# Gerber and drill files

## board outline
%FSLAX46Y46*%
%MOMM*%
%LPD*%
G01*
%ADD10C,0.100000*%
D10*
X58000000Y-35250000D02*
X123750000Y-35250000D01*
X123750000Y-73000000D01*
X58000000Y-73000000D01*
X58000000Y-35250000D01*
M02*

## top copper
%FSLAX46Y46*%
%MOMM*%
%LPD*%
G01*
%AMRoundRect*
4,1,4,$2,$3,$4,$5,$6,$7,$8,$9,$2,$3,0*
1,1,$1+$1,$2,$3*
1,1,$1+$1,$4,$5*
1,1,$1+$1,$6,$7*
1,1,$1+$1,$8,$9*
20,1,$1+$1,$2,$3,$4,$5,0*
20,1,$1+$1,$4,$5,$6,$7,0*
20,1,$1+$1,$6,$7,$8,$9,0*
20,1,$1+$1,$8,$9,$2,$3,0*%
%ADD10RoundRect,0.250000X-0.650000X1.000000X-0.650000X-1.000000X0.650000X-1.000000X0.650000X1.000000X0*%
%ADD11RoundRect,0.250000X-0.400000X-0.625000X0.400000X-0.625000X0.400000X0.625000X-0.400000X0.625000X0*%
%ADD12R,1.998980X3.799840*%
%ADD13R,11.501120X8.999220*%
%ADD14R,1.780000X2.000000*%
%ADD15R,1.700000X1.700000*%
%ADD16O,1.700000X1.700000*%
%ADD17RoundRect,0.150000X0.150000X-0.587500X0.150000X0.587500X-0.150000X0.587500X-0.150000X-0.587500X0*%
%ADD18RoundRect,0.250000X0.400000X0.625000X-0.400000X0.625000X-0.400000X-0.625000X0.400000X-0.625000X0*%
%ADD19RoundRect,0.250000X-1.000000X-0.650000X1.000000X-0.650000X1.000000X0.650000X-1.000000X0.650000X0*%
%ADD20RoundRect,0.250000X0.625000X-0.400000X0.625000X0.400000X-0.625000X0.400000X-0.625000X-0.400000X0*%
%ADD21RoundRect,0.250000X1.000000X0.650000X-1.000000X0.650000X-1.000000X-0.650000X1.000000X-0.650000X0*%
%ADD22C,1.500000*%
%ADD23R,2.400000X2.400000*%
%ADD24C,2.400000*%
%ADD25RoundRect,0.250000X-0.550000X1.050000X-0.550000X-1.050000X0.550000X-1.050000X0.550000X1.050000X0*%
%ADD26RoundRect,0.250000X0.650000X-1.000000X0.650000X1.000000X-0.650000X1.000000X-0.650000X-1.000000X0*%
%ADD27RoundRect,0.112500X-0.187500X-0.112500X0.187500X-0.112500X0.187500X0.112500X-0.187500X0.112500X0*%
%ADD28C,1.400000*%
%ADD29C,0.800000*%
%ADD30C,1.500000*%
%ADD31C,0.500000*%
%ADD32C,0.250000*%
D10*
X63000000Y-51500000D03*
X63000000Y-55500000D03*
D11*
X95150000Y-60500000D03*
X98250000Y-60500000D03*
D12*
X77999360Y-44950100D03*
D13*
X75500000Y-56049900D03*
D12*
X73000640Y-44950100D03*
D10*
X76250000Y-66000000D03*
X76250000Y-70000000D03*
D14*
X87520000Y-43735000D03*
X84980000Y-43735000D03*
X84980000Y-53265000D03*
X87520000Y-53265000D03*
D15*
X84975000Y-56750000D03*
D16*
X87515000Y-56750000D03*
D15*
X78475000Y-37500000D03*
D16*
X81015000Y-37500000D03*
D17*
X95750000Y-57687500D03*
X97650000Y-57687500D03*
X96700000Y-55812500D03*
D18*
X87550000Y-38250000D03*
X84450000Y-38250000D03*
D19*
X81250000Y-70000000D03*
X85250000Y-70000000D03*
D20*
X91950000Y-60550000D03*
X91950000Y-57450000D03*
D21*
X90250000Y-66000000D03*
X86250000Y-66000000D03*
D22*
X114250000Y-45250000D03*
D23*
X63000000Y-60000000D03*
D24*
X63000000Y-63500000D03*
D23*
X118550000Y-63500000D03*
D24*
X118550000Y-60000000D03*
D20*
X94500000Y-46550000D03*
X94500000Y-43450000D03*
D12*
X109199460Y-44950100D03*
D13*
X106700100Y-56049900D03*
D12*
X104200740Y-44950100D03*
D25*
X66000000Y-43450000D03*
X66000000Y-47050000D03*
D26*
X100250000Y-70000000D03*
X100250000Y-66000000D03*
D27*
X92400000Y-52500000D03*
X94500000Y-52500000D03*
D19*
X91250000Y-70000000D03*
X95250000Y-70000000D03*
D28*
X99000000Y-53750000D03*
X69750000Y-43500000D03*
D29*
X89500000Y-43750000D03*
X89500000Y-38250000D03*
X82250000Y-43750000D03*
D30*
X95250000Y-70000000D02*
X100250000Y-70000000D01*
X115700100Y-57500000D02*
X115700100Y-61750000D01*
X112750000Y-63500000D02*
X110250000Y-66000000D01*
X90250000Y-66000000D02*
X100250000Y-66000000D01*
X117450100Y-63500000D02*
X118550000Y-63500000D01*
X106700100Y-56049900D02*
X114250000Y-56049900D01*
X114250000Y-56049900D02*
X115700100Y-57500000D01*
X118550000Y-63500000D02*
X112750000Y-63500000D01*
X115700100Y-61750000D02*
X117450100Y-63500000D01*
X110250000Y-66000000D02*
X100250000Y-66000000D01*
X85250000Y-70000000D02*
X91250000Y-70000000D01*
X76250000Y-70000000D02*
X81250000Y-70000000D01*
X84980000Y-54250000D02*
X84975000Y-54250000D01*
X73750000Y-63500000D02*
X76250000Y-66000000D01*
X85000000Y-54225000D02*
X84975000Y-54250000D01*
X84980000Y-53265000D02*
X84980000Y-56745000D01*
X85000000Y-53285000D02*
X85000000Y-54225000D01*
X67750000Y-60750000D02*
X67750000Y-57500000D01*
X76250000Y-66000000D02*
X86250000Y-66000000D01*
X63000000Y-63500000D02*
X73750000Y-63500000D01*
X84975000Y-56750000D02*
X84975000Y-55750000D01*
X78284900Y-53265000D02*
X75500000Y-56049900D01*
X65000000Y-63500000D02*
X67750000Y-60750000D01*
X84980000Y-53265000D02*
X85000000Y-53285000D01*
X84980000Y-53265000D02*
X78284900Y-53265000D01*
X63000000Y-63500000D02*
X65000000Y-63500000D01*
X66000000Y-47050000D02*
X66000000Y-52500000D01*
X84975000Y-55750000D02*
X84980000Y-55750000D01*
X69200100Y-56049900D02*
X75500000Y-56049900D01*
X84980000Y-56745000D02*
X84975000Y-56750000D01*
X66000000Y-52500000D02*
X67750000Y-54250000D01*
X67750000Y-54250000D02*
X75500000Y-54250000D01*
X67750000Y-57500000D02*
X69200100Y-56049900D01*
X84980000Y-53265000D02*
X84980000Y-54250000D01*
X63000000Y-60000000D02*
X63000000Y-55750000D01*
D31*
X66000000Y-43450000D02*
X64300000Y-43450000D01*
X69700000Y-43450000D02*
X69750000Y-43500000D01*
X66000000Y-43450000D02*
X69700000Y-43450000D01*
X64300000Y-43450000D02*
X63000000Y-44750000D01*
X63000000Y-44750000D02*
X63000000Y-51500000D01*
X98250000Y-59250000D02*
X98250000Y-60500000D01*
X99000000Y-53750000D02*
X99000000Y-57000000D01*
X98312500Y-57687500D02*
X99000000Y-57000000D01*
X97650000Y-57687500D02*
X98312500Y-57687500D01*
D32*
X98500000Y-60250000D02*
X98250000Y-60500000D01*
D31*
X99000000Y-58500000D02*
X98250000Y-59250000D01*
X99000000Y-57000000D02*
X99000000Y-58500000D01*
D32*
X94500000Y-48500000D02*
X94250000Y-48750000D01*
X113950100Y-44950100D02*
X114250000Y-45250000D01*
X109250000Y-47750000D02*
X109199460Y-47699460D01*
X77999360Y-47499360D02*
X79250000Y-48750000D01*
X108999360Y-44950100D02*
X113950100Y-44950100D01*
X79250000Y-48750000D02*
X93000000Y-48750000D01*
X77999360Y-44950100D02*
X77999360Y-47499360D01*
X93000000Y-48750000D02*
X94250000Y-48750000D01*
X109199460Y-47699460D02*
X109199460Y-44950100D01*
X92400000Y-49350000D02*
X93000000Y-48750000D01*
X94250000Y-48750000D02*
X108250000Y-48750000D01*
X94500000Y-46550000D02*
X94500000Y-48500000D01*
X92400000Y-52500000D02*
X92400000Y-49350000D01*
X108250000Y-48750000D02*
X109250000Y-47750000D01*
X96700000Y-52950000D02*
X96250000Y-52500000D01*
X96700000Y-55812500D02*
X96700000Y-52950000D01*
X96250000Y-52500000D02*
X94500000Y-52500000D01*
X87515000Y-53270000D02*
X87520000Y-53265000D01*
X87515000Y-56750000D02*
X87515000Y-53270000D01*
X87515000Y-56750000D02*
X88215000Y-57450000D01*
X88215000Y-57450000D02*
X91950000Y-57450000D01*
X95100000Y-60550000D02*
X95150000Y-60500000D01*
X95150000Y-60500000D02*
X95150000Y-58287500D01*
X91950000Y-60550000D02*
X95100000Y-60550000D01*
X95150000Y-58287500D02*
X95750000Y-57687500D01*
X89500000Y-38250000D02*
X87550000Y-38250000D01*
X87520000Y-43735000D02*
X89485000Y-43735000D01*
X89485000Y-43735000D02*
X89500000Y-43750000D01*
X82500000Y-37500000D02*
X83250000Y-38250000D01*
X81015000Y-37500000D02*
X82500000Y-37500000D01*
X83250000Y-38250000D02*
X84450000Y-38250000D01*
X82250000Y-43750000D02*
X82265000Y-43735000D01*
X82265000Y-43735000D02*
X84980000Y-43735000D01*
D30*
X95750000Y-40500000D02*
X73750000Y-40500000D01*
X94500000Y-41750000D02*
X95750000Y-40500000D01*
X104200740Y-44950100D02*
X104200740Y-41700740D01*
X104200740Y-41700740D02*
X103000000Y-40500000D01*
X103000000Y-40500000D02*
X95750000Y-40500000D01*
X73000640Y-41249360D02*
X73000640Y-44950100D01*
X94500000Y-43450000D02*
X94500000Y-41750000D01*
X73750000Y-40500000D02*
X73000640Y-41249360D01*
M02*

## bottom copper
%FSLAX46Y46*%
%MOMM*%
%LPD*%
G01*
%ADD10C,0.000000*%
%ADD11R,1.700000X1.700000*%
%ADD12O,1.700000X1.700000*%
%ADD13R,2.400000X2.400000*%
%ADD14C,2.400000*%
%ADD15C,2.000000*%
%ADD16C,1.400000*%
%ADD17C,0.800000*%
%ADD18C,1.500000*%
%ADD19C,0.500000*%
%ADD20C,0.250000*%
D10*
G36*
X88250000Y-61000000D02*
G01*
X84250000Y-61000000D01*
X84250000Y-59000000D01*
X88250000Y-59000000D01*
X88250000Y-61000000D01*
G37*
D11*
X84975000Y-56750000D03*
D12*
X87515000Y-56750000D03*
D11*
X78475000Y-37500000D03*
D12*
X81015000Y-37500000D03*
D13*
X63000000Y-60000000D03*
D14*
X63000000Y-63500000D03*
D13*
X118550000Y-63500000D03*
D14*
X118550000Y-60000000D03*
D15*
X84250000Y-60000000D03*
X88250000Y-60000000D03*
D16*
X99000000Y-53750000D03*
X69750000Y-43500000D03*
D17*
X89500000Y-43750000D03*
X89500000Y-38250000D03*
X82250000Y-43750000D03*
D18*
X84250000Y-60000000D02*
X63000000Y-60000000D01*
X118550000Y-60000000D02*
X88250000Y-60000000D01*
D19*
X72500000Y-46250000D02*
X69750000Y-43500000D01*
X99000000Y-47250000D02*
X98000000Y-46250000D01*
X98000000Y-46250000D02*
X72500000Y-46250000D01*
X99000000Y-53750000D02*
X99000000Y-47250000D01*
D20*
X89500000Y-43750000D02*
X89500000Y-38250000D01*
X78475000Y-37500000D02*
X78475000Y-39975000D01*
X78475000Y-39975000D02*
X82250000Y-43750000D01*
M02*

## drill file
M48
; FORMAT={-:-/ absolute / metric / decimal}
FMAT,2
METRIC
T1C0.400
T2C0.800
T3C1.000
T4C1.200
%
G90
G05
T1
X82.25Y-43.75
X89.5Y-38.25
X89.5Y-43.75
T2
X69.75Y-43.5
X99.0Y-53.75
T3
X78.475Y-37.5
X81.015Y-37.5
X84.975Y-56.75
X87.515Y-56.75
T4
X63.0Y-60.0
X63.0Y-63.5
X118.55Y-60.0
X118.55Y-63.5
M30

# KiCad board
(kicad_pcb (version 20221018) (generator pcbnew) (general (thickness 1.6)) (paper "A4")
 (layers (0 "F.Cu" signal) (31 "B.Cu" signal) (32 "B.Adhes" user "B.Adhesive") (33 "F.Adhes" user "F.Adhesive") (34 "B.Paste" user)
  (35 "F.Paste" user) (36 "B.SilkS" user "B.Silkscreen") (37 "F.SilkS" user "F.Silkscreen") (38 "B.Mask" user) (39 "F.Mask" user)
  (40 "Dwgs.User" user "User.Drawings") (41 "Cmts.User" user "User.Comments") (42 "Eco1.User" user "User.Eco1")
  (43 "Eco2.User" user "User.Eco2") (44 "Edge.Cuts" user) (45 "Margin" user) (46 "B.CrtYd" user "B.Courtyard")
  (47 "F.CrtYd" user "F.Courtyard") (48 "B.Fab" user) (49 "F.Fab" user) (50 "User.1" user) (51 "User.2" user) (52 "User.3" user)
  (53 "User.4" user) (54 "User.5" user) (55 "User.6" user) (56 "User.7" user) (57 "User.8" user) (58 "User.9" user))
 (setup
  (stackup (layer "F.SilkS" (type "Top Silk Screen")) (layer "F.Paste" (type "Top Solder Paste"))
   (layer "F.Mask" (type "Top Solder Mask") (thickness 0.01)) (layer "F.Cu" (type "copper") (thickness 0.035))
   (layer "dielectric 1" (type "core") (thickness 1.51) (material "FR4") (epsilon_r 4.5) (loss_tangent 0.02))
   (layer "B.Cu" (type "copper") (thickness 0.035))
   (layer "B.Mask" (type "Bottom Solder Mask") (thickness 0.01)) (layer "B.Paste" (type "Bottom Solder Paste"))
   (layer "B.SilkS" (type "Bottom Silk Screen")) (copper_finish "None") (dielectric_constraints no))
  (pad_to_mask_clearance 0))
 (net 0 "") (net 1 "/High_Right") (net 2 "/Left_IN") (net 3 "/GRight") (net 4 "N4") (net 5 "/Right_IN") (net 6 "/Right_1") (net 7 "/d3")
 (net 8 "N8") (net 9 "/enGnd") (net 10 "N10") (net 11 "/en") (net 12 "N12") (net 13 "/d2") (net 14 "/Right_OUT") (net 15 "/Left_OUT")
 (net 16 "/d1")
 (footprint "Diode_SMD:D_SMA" (layer "F.Cu") (at 63 53.5 -90)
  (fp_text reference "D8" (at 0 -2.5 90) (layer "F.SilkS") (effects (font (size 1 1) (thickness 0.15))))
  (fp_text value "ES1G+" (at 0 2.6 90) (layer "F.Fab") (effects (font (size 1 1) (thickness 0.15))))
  (pad "1" smd roundrect (at -2 0 270) (size 2.5 1.8) (layers "F.Cu" "F.Paste" "F.Mask") (roundrect_rratio 0.1388888889)
   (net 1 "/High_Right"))
  (pad "2" smd roundrect (at 2 0 270) (size 2.5 1.8) (layers "F.Cu" "F.Paste" "F.Mask") (roundrect_rratio 0.1388888889) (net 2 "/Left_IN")))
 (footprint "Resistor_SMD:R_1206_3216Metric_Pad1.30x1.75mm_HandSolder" (layer "F.Cu") (at 96.7 60.5)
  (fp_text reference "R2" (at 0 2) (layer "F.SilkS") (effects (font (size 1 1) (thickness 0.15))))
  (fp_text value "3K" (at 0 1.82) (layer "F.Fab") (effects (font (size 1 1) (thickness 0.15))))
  (pad "1" smd roundrect (at -1.55 0) (size 1.3 1.75) (layers "F.Cu" "F.Paste" "F.Mask") (roundrect_rratio 0.192308) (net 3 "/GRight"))
  (pad "2" smd roundrect (at 1.55 0) (size 1.3 1.75) (layers "F.Cu" "F.Paste" "F.Mask") (roundrect_rratio 0.192308) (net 1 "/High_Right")))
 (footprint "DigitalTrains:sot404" (layer "F.Cu") (at 75.5 50.5 180)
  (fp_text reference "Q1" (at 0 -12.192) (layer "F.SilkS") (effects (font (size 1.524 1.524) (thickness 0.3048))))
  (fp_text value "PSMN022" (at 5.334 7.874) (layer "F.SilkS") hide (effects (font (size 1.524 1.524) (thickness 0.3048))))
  (pad "1" smd rect (at -2.49936 5.5499 180) (size 1.99898 3.79984) (layers "F.Cu" "F.Paste" "F.Mask") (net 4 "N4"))
  (pad "2" smd rect (at 0 -5.5499 180) (size 11.50112 8.99922) (layers "F.Cu" "F.Paste" "F.Mask") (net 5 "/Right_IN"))
  (pad "3" smd rect (at 2.49936 5.5499 180) (size 1.99898 3.79984) (layers "F.Cu" "F.Paste" "F.Mask") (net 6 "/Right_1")))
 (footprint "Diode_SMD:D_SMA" (layer "F.Cu") (at 76.25 68 -90)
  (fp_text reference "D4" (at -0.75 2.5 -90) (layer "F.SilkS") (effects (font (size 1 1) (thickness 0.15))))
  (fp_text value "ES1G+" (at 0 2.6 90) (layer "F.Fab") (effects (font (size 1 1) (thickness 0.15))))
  (pad "1" smd roundrect (at -2 0 270) (size 2.5 1.8) (layers "F.Cu" "F.Paste" "F.Mask") (roundrect_rratio 0.1388888889) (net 5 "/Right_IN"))
  (pad "2" smd roundrect (at 2 0 270) (size 2.5 1.8) (layers "F.Cu" "F.Paste" "F.Mask") (roundrect_rratio 0.1388888889) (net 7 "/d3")))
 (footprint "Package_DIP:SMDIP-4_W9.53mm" (layer "F.Cu") (at 86.25 48.5 -90)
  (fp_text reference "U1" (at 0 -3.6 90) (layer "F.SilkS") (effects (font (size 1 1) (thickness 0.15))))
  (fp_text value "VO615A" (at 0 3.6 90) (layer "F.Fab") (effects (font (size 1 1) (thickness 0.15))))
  (pad "1" smd rect (at -4.765 -1.27 270) (size 2 1.78) (layers "F.Cu" "F.Paste" "F.Mask") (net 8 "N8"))
  (pad "2" smd rect (at -4.765 1.27 270) (size 2 1.78) (layers "F.Cu" "F.Paste" "F.Mask") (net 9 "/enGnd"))
  (pad "3" smd rect (at 4.765 1.27 270) (size 2 1.78) (layers "F.Cu" "F.Paste" "F.Mask") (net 5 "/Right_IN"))
  (pad "4" smd rect (at 4.765 -1.27 270) (size 2 1.78) (layers "F.Cu" "F.Paste" "F.Mask") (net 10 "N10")))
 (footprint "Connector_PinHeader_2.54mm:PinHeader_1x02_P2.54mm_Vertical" (layer "F.Cu") (at 84.975 56.75 90) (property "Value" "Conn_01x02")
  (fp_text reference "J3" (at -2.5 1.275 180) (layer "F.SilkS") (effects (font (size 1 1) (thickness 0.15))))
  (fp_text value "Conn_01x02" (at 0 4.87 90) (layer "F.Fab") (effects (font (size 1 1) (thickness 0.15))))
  (pad "1" thru_hole rect (at 0 0 90) (size 1.7 1.7) (drill 1) (layers "*.Cu" "*.Mask") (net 5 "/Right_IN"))
  (pad "2" thru_hole oval (at 0 2.54 90) (size 1.7 1.7) (drill 1) (layers "*.Cu" "*.Mask") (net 10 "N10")))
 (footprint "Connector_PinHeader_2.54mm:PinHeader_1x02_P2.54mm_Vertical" (layer "F.Cu") (at 78.475 37.5 90) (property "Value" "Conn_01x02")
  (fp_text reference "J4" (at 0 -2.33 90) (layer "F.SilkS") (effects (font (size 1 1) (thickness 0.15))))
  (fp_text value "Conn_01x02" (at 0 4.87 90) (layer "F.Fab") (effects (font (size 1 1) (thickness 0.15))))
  (pad "1" thru_hole rect (at 0 0 90) (size 1.7 1.7) (drill 1) (layers "*.Cu" "*.Mask") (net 9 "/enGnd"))
  (pad "2" thru_hole oval (at 0 2.54 90) (size 1.7 1.7) (drill 1) (layers "*.Cu" "*.Mask") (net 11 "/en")))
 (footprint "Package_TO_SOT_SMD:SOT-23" (layer "F.Cu") (at 96.7 56.75 90)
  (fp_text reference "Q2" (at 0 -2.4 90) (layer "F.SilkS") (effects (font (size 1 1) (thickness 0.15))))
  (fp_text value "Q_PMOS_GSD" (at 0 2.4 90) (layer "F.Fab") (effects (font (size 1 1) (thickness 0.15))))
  (pad "1" smd roundrect (at -0.9375 -0.95 90) (size 1.475 0.6) (layers "F.Cu" "F.Paste" "F.Mask") (roundrect_rratio 0.25) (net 3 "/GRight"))
  (pad "2" smd roundrect (at -0.9375 0.95 90) (size 1.475 0.6) (layers "F.Cu" "F.Paste" "F.Mask") (roundrect_rratio 0.25)
   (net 1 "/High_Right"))
  (pad "3" smd roundrect (at 0.9375 0 90) (size 1.475 0.6) (layers "F.Cu" "F.Paste" "F.Mask") (roundrect_rratio 0.25) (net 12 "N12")))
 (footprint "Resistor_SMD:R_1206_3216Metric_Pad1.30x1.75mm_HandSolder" (layer "F.Cu") (at 86 38.25 180)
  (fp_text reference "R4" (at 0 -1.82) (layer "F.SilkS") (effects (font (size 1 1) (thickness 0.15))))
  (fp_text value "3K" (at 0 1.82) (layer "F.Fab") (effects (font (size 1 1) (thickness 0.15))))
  (pad "1" smd roundrect (at -1.55 0 180) (size 1.3 1.75) (layers "F.Cu" "F.Paste" "F.Mask") (roundrect_rratio 0.192308) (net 8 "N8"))
  (pad "2" smd roundrect (at 1.55 0 180) (size 1.3 1.75) (layers "F.Cu" "F.Paste" "F.Mask") (roundrect_rratio 0.192308) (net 11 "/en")))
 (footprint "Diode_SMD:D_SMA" (layer "F.Cu") (at 83.25 70)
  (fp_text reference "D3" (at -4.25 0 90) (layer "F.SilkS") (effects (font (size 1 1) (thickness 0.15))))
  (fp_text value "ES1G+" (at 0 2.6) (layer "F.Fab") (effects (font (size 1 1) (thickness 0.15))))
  (pad "1" smd roundrect (at -2 0) (size 2.5 1.8) (layers "F.Cu" "F.Paste" "F.Mask") (roundrect_rratio 0.1388888889) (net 7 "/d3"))
  (pad "2" smd roundrect (at 2 0) (size 2.5 1.8) (layers "F.Cu" "F.Paste" "F.Mask") (roundrect_rratio 0.1388888889) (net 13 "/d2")))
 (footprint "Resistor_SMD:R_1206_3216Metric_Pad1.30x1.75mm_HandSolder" (layer "F.Cu") (at 91.95 59 90)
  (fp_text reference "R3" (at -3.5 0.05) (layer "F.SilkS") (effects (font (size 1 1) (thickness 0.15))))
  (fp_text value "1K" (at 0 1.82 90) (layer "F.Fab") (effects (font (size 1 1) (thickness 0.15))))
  (pad "1" smd roundrect (at -1.55 0 90) (size 1.3 1.75) (layers "F.Cu" "F.Paste" "F.Mask") (roundrect_rratio 0.192308) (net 3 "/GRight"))
  (pad "2" smd roundrect (at 1.55 0 90) (size 1.3 1.75) (layers "F.Cu" "F.Paste" "F.Mask") (roundrect_rratio 0.192308) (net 10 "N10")))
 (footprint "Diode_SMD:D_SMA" (layer "F.Cu") (at 88.25 66 180)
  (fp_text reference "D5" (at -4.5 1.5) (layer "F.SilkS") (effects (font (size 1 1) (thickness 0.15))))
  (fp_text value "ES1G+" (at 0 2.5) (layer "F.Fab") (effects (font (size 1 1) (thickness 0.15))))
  (pad "1" smd roundrect (at -2 0 180) (size 2.5 1.8) (layers "F.Cu" "F.Paste" "F.Mask") (roundrect_rratio 0.1388888889)
   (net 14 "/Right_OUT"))
  (pad "2" smd roundrect (at 2 0 180) (size 2.5 1.8) (layers "F.Cu" "F.Paste" "F.Mask") (roundrect_rratio 0.1388888889) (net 5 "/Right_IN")))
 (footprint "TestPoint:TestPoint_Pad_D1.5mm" (layer "F.Cu") (at 114.25 45.25)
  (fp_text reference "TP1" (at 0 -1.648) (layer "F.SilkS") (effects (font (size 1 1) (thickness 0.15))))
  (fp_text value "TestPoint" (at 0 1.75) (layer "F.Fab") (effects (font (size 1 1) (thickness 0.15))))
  (pad "1" smd circle (at 0 0) (size 1.5 1.5) (layers "F.Cu" "F.Mask") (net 4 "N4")))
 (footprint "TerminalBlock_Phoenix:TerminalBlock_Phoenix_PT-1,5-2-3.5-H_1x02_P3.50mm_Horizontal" (layer "F.Cu") (at 63 60 -90)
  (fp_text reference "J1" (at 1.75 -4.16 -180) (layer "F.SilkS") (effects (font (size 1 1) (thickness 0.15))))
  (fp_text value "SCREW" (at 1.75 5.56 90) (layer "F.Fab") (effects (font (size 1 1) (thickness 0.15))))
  (pad "1" thru_hole rect (at 0 0 270) (size 2.4 2.4) (drill 1.2) (layers "*.Cu" "*.Mask") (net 2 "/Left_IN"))
  (pad "2" thru_hole circle (at 3.5 0 270) (size 2.4 2.4) (drill 1.2) (layers "*.Cu" "*.Mask") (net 5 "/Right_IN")))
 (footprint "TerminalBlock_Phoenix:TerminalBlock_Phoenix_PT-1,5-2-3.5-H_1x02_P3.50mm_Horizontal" (layer "F.Cu") (at 118.55 63.5 90)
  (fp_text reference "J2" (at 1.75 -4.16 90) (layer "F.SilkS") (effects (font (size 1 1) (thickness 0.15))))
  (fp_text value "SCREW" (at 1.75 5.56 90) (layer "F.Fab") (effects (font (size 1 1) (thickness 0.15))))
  (pad "1" thru_hole rect (at 0 0 90) (size 2.4 2.4) (drill 1.2) (layers "*.Cu" "*.Mask") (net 14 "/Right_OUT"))
  (pad "2" thru_hole circle (at 3.5 0 90) (size 2.4 2.4) (drill 1.2) (layers "*.Cu" "*.Mask") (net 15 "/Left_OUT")))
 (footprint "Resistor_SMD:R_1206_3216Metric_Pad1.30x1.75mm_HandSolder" (layer "F.Cu") (at 94.5 45 90)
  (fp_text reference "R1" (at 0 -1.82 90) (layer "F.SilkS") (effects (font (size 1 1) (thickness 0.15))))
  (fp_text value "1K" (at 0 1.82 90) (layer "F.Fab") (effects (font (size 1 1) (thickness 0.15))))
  (pad "1" smd roundrect (at -1.55 0 90) (size 1.3 1.75) (layers "F.Cu" "F.Paste" "F.Mask") (roundrect_rratio 0.192308) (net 4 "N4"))
  (pad "2" smd roundrect (at 1.55 0 90) (size 1.3 1.75) (layers "F.Cu" "F.Paste" "F.Mask") (roundrect_rratio 0.192308) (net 6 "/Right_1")))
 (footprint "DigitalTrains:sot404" (layer "F.Cu") (at 106.7001 50.5 180)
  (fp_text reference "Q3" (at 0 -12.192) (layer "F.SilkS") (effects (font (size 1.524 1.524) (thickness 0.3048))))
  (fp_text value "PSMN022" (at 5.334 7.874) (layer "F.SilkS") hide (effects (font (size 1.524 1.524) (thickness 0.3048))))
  (pad "1" smd rect (at -2.49936 5.5499 180) (size 1.99898 3.79984) (layers "F.Cu" "F.Paste" "F.Mask") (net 4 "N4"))
  (pad "2" smd rect (at 0 -5.5499 180) (size 11.50112 8.99922) (layers "F.Cu" "F.Paste" "F.Mask") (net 14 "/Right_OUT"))
  (pad "3" smd rect (at 2.49936 5.5499 180) (size 1.99898 3.79984) (layers "F.Cu" "F.Paste" "F.Mask") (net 6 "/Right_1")))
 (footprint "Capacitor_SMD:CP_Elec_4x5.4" (layer "F.Cu") (at 66 45.25 -90)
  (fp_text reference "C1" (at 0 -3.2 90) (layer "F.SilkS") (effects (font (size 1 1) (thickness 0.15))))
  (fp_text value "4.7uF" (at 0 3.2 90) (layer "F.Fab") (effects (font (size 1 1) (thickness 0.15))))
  (pad "1" smd roundrect (at -1.8 0 270) (size 2.6 1.6) (layers "F.Cu" "F.Paste" "F.Mask") (roundrect_rratio 0.15625) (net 1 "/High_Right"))
  (pad "2" smd roundrect (at 1.8 0 270) (size 2.6 1.6) (layers "F.Cu" "F.Paste" "F.Mask") (roundrect_rratio 0.15625) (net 5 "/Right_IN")))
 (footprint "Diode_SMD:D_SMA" (layer "F.Cu") (at 100.25 68 90)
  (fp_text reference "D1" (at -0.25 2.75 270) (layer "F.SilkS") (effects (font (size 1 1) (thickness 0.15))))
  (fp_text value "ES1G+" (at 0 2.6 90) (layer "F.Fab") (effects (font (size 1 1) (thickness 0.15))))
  (pad "1" smd roundrect (at -2 0 90) (size 2.5 1.8) (layers "F.Cu" "F.Paste" "F.Mask") (roundrect_rratio 0.1388888889) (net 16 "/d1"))
  (pad "2" smd roundrect (at 2 0 90) (size 2.5 1.8) (layers "F.Cu" "F.Paste" "F.Mask") (roundrect_rratio 0.1388888889) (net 14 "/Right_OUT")))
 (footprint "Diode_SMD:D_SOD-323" (layer "F.Cu") (at 93.45 52.5)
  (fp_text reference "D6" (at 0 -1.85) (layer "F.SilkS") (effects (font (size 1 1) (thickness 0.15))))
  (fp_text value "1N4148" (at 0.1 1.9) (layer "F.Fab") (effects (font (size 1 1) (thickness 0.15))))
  (pad "1" smd roundrect (at -1.05 0) (size 0.6 0.45) (layers "F.Cu" "F.Paste" "F.Mask") (roundrect_rratio 0.25) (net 4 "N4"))
  (pad "2" smd roundrect (at 1.05 0) (size 0.6 0.45) (layers "F.Cu" "F.Paste" "F.Mask") (roundrect_rratio 0.25) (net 12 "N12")))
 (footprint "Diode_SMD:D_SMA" (layer "F.Cu") (at 93.25 70)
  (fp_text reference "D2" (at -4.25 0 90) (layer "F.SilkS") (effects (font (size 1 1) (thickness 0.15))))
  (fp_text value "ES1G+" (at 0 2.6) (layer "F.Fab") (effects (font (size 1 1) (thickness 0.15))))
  (pad "1" smd roundrect (at -2 0) (size 2.5 1.8) (layers "F.Cu" "F.Paste" "F.Mask") (roundrect_rratio 0.1388888889) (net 13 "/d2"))
  (pad "2" smd roundrect (at 2 0) (size 2.5 1.8) (layers "F.Cu" "F.Paste" "F.Mask") (roundrect_rratio 0.1388888889) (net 16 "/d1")))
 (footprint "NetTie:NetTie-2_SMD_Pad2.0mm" (layer "B.Cu") (at 86.25 60) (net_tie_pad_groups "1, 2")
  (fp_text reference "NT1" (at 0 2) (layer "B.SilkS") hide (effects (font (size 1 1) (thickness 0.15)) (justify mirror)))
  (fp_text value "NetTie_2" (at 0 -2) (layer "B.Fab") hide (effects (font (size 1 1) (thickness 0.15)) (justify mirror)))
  (fp_poly (pts (xy -2 1) (xy 2 1) (xy 2 -1) (xy -2 -1)) (stroke (width 0) (type solid)) (fill solid) (layer "B.Cu"))
  (pad "1" smd circle (at -2 0) (size 2 2) (layers "B.Cu") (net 2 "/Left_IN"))
  (pad "2" smd circle (at 2 0) (size 2 2) (layers "B.Cu") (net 15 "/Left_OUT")))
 (gr_rect (start 58 35.25) (end 123.75 73) (stroke (width 0.1) (type default)) (fill none) (layer "Edge.Cuts"))
 (segment (start 95.25 70) (end 100.25 70) (width 1.5) (layer "F.Cu") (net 16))
 (segment (start 115.7001 57.5) (end 115.7001 61.75) (width 1.5) (layer "F.Cu") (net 14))
 (segment (start 112.75 63.5) (end 110.25 66) (width 1.5) (layer "F.Cu") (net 14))
 (segment (start 90.25 66) (end 100.25 66) (width 1.5) (layer "F.Cu") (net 14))
 (segment (start 117.4501 63.5) (end 118.55 63.5) (width 1.5) (layer "F.Cu") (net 14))
 (segment (start 106.7001 56.0499) (end 114.25 56.0499) (width 1.5) (layer "F.Cu") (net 14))
 (segment (start 114.25 56.0499) (end 115.7001 57.5) (width 1.5) (layer "F.Cu") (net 14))
 (segment (start 118.55 63.5) (end 112.75 63.5) (width 1.5) (layer "F.Cu") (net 14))
 (segment (start 115.7001 61.75) (end 117.4501 63.5) (width 1.5) (layer "F.Cu") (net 14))
 (segment (start 110.25 66) (end 100.25 66) (width 1.5) (layer "F.Cu") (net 14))
 (segment (start 85.25 70) (end 91.25 70) (width 1.5) (layer "F.Cu") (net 13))
 (segment (start 76.25 70) (end 81.25 70) (width 1.5) (layer "F.Cu") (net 7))
 (segment (start 84.98 54.25) (end 84.975 54.25) (width 1.5) (layer "F.Cu") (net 5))
 (segment (start 73.75 63.5) (end 76.25 66) (width 1.5) (layer "F.Cu") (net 5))
 (segment (start 85 54.225) (end 84.975 54.25) (width 1.5) (layer "F.Cu") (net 5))
 (segment (start 84.98 53.265) (end 84.98 56.745) (width 1.5) (layer "F.Cu") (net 5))
 (segment (start 85 53.285) (end 85 54.225) (width 1.5) (layer "F.Cu") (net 5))
 (segment (start 67.75 60.75) (end 67.75 57.5) (width 1.5) (layer "F.Cu") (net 5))
 (segment (start 76.25 66) (end 86.25 66) (width 1.5) (layer "F.Cu") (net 5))
 (segment (start 63 63.5) (end 73.75 63.5) (width 1.5) (layer "F.Cu") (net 5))
 (segment (start 84.975 56.75) (end 84.975 55.75) (width 1.5) (layer "F.Cu") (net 5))
 (segment (start 78.2849 53.265) (end 75.5 56.0499) (width 1.5) (layer "F.Cu") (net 5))
 (segment (start 65 63.5) (end 67.75 60.75) (width 1.5) (layer "F.Cu") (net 5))
 (segment (start 84.98 53.265) (end 85 53.285) (width 1.5) (layer "F.Cu") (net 5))
 (segment (start 84.98 53.265) (end 78.2849 53.265) (width 1.5) (layer "F.Cu") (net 5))
 (segment (start 63 63.5) (end 65 63.5) (width 1.5) (layer "F.Cu") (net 5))
 (segment (start 66 47.05) (end 66 52.5) (width 1.5) (layer "F.Cu") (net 5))
 (segment (start 84.975 55.75) (end 84.98 55.75) (width 1.5) (layer "F.Cu") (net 5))
 (segment (start 69.2001 56.0499) (end 75.5 56.0499) (width 1.5) (layer "F.Cu") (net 5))
 (segment (start 84.98 56.745) (end 84.975 56.75) (width 1.5) (layer "F.Cu") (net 5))
 (segment (start 66 52.5) (end 67.75 54.25) (width 1.5) (layer "F.Cu") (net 5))
 (segment (start 67.75 54.25) (end 75.5 54.25) (width 1.5) (layer "F.Cu") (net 5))
 (segment (start 67.75 57.5) (end 69.2001 56.0499) (width 1.5) (layer "F.Cu") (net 5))
 (segment (start 84.98 53.265) (end 84.98 54.25) (width 1.5) (layer "F.Cu") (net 5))
 (segment (start 63 60) (end 63 55.75) (width 1.5) (layer "F.Cu") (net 2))
 (segment (start 84.25 60) (end 63 60) (width 1.5) (layer "B.Cu") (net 2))
 (segment (start 118.55 60) (end 88.25 60) (width 1.5) (layer "B.Cu") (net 15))
 (segment (start 66 43.45) (end 64.3 43.45) (width 0.5) (layer "F.Cu") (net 1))
 (segment (start 69.7 43.45) (end 69.75 43.5) (width 0.5) (layer "F.Cu") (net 1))
 (segment (start 66 43.45) (end 69.7 43.45) (width 0.5) (layer "F.Cu") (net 1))
 (segment (start 64.3 43.45) (end 63 44.75) (width 0.5) (layer "F.Cu") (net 1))
 (segment (start 63 44.75) (end 63 51.5) (width 0.5) (layer "F.Cu") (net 1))
 (segment (start 98.25 59.25) (end 98.25 60.5) (width 0.5) (layer "F.Cu") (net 1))
 (segment (start 99 53.75) (end 99 57) (width 0.5) (layer "F.Cu") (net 1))
 (segment (start 98.3125 57.6875) (end 99 57) (width 0.5) (layer "F.Cu") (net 1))
 (segment (start 97.65 57.6875) (end 98.3125 57.6875) (width 0.5) (layer "F.Cu") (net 1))
 (segment (start 98.5 60.25) (end 98.25 60.5) (width 0.25) (layer "F.Cu") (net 1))
 (segment (start 99 58.5) (end 98.25 59.25) (width 0.5) (layer "F.Cu") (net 1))
 (segment (start 99 57) (end 99 58.5) (width 0.5) (layer "F.Cu") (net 1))
 (via (at 99 53.75) (size 1.4) (drill 0.8) (layers "F.Cu" "B.Cu") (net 1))
 (via (at 69.75 43.5) (size 1.4) (drill 0.8) (layers "F.Cu" "B.Cu") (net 1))
 (segment (start 72.5 46.25) (end 69.75 43.5) (width 0.5) (layer "B.Cu") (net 1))
 (segment (start 99 47.25) (end 98 46.25) (width 0.5) (layer "B.Cu") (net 1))
 (segment (start 98 46.25) (end 72.5 46.25) (width 0.5) (layer "B.Cu") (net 1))
 (segment (start 99 53.75) (end 99 47.25) (width 0.5) (layer "B.Cu") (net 1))
 (segment (start 94.5 48.5) (end 94.25 48.75) (width 0.25) (layer "F.Cu") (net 4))
 (segment (start 113.9501 44.9501) (end 114.25 45.25) (width 0.25) (layer "F.Cu") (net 4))
 (segment (start 109.25 47.75) (end 109.19946 47.69946) (width 0.25) (layer "F.Cu") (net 4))
 (segment (start 77.99936 47.49936) (end 79.25 48.75) (width 0.25) (layer "F.Cu") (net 4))
 (segment (start 108.99936 44.9501) (end 113.9501 44.9501) (width 0.25) (layer "F.Cu") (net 4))
 (segment (start 79.25 48.75) (end 93 48.75) (width 0.25) (layer "F.Cu") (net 4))
 (segment (start 77.99936 44.9501) (end 77.99936 47.49936) (width 0.25) (layer "F.Cu") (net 4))
 (segment (start 93 48.75) (end 94.25 48.75) (width 0.25) (layer "F.Cu") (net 4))
 (segment (start 109.19946 47.69946) (end 109.19946 44.9501) (width 0.25) (layer "F.Cu") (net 4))
 (segment (start 92.4 49.35) (end 93 48.75) (width 0.25) (layer "F.Cu") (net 4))
 (segment (start 94.25 48.75) (end 108.25 48.75) (width 0.25) (layer "F.Cu") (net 4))
 (segment (start 94.5 46.55) (end 94.5 48.5) (width 0.25) (layer "F.Cu") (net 4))
 (segment (start 92.4 52.5) (end 92.4 49.35) (width 0.25) (layer "F.Cu") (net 4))
 (segment (start 108.25 48.75) (end 109.25 47.75) (width 0.25) (layer "F.Cu") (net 4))
 (segment (start 96.7 52.95) (end 96.25 52.5) (width 0.25) (layer "F.Cu") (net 12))
 (segment (start 96.7 55.8125) (end 96.7 52.95) (width 0.25) (layer "F.Cu") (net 12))
 (segment (start 96.25 52.5) (end 94.5 52.5) (width 0.25) (layer "F.Cu") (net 12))
 (segment (start 87.515 53.27) (end 87.52 53.265) (width 0.25) (layer "F.Cu") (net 10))
 (segment (start 87.515 56.75) (end 87.515 53.27) (width 0.25) (layer "F.Cu") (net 10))
 (segment (start 87.515 56.75) (end 88.215 57.45) (width 0.25) (layer "F.Cu") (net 10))
 (segment (start 88.215 57.45) (end 91.95 57.45) (width 0.25) (layer "F.Cu") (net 10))
 (segment (start 95.1 60.55) (end 95.15 60.5) (width 0.25) (layer "F.Cu") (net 3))
 (segment (start 95.15 60.5) (end 95.15 58.2875) (width 0.25) (layer "F.Cu") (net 3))
 (segment (start 91.95 60.55) (end 95.1 60.55) (width 0.25) (layer "F.Cu") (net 3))
 (segment (start 95.15 58.2875) (end 95.75 57.6875) (width 0.25) (layer "F.Cu") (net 3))
 (segment (start 89.5 38.25) (end 87.55 38.25) (width 0.25) (layer "F.Cu") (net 8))
 (segment (start 87.52 43.735) (end 89.485 43.735) (width 0.25) (layer "F.Cu") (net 8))
 (segment (start 89.485 43.735) (end 89.5 43.75) (width 0.25) (layer "F.Cu") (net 8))
 (via (at 89.5 43.75) (size 0.8) (drill 0.4) (layers "F.Cu" "B.Cu") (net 8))
 (via (at 89.5 38.25) (size 0.8) (drill 0.4) (layers "F.Cu" "B.Cu") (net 8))
 (segment (start 89.5 43.75) (end 89.5 38.25) (width 0.25) (layer "B.Cu") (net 8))
 (segment (start 82.5 37.5) (end 83.25 38.25) (width 0.25) (layer "F.Cu") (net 11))
 (segment (start 81.015 37.5) (end 82.5 37.5) (width 0.25) (layer "F.Cu") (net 11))
 (segment (start 83.25 38.25) (end 84.45 38.25) (width 0.25) (layer "F.Cu") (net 11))
 (segment (start 82.25 43.75) (end 82.265 43.735) (width 0.25) (layer "F.Cu") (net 9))
 (segment (start 82.265 43.735) (end 84.98 43.735) (width 0.25) (layer "F.Cu") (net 9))
 (via (at 82.25 43.75) (size 0.8) (drill 0.4) (layers "F.Cu" "B.Cu") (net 9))
 (segment (start 78.475 37.5) (end 78.475 39.975) (width 0.25) (layer "B.Cu") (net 9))
 (segment (start 78.475 39.975) (end 82.25 43.75) (width 0.25) (layer "B.Cu") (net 9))
 (segment (start 95.75 40.5) (end 73.75 40.5) (width 1.5) (layer "F.Cu") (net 6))
 (segment (start 94.5 41.75) (end 95.75 40.5) (width 1.5) (layer "F.Cu") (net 6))
 (segment (start 104.20074 44.9501) (end 104.20074 41.70074) (width 1.5) (layer "F.Cu") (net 6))
 (segment (start 104.20074 41.70074) (end 103 40.5) (width 1.5) (layer "F.Cu") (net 6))
 (segment (start 103 40.5) (end 95.75 40.5) (width 1.5) (layer "F.Cu") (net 6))
 (segment (start 73.00064 41.24936) (end 73.00064 44.9501) (width 1.5) (layer "F.Cu") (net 6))
 (segment (start 94.5 43.45) (end 94.5 41.75) (width 1.5) (layer "F.Cu") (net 6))
 (segment (start 73.75 40.5) (end 73.00064 41.24936) (width 1.5) (layer "F.Cu") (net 6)))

